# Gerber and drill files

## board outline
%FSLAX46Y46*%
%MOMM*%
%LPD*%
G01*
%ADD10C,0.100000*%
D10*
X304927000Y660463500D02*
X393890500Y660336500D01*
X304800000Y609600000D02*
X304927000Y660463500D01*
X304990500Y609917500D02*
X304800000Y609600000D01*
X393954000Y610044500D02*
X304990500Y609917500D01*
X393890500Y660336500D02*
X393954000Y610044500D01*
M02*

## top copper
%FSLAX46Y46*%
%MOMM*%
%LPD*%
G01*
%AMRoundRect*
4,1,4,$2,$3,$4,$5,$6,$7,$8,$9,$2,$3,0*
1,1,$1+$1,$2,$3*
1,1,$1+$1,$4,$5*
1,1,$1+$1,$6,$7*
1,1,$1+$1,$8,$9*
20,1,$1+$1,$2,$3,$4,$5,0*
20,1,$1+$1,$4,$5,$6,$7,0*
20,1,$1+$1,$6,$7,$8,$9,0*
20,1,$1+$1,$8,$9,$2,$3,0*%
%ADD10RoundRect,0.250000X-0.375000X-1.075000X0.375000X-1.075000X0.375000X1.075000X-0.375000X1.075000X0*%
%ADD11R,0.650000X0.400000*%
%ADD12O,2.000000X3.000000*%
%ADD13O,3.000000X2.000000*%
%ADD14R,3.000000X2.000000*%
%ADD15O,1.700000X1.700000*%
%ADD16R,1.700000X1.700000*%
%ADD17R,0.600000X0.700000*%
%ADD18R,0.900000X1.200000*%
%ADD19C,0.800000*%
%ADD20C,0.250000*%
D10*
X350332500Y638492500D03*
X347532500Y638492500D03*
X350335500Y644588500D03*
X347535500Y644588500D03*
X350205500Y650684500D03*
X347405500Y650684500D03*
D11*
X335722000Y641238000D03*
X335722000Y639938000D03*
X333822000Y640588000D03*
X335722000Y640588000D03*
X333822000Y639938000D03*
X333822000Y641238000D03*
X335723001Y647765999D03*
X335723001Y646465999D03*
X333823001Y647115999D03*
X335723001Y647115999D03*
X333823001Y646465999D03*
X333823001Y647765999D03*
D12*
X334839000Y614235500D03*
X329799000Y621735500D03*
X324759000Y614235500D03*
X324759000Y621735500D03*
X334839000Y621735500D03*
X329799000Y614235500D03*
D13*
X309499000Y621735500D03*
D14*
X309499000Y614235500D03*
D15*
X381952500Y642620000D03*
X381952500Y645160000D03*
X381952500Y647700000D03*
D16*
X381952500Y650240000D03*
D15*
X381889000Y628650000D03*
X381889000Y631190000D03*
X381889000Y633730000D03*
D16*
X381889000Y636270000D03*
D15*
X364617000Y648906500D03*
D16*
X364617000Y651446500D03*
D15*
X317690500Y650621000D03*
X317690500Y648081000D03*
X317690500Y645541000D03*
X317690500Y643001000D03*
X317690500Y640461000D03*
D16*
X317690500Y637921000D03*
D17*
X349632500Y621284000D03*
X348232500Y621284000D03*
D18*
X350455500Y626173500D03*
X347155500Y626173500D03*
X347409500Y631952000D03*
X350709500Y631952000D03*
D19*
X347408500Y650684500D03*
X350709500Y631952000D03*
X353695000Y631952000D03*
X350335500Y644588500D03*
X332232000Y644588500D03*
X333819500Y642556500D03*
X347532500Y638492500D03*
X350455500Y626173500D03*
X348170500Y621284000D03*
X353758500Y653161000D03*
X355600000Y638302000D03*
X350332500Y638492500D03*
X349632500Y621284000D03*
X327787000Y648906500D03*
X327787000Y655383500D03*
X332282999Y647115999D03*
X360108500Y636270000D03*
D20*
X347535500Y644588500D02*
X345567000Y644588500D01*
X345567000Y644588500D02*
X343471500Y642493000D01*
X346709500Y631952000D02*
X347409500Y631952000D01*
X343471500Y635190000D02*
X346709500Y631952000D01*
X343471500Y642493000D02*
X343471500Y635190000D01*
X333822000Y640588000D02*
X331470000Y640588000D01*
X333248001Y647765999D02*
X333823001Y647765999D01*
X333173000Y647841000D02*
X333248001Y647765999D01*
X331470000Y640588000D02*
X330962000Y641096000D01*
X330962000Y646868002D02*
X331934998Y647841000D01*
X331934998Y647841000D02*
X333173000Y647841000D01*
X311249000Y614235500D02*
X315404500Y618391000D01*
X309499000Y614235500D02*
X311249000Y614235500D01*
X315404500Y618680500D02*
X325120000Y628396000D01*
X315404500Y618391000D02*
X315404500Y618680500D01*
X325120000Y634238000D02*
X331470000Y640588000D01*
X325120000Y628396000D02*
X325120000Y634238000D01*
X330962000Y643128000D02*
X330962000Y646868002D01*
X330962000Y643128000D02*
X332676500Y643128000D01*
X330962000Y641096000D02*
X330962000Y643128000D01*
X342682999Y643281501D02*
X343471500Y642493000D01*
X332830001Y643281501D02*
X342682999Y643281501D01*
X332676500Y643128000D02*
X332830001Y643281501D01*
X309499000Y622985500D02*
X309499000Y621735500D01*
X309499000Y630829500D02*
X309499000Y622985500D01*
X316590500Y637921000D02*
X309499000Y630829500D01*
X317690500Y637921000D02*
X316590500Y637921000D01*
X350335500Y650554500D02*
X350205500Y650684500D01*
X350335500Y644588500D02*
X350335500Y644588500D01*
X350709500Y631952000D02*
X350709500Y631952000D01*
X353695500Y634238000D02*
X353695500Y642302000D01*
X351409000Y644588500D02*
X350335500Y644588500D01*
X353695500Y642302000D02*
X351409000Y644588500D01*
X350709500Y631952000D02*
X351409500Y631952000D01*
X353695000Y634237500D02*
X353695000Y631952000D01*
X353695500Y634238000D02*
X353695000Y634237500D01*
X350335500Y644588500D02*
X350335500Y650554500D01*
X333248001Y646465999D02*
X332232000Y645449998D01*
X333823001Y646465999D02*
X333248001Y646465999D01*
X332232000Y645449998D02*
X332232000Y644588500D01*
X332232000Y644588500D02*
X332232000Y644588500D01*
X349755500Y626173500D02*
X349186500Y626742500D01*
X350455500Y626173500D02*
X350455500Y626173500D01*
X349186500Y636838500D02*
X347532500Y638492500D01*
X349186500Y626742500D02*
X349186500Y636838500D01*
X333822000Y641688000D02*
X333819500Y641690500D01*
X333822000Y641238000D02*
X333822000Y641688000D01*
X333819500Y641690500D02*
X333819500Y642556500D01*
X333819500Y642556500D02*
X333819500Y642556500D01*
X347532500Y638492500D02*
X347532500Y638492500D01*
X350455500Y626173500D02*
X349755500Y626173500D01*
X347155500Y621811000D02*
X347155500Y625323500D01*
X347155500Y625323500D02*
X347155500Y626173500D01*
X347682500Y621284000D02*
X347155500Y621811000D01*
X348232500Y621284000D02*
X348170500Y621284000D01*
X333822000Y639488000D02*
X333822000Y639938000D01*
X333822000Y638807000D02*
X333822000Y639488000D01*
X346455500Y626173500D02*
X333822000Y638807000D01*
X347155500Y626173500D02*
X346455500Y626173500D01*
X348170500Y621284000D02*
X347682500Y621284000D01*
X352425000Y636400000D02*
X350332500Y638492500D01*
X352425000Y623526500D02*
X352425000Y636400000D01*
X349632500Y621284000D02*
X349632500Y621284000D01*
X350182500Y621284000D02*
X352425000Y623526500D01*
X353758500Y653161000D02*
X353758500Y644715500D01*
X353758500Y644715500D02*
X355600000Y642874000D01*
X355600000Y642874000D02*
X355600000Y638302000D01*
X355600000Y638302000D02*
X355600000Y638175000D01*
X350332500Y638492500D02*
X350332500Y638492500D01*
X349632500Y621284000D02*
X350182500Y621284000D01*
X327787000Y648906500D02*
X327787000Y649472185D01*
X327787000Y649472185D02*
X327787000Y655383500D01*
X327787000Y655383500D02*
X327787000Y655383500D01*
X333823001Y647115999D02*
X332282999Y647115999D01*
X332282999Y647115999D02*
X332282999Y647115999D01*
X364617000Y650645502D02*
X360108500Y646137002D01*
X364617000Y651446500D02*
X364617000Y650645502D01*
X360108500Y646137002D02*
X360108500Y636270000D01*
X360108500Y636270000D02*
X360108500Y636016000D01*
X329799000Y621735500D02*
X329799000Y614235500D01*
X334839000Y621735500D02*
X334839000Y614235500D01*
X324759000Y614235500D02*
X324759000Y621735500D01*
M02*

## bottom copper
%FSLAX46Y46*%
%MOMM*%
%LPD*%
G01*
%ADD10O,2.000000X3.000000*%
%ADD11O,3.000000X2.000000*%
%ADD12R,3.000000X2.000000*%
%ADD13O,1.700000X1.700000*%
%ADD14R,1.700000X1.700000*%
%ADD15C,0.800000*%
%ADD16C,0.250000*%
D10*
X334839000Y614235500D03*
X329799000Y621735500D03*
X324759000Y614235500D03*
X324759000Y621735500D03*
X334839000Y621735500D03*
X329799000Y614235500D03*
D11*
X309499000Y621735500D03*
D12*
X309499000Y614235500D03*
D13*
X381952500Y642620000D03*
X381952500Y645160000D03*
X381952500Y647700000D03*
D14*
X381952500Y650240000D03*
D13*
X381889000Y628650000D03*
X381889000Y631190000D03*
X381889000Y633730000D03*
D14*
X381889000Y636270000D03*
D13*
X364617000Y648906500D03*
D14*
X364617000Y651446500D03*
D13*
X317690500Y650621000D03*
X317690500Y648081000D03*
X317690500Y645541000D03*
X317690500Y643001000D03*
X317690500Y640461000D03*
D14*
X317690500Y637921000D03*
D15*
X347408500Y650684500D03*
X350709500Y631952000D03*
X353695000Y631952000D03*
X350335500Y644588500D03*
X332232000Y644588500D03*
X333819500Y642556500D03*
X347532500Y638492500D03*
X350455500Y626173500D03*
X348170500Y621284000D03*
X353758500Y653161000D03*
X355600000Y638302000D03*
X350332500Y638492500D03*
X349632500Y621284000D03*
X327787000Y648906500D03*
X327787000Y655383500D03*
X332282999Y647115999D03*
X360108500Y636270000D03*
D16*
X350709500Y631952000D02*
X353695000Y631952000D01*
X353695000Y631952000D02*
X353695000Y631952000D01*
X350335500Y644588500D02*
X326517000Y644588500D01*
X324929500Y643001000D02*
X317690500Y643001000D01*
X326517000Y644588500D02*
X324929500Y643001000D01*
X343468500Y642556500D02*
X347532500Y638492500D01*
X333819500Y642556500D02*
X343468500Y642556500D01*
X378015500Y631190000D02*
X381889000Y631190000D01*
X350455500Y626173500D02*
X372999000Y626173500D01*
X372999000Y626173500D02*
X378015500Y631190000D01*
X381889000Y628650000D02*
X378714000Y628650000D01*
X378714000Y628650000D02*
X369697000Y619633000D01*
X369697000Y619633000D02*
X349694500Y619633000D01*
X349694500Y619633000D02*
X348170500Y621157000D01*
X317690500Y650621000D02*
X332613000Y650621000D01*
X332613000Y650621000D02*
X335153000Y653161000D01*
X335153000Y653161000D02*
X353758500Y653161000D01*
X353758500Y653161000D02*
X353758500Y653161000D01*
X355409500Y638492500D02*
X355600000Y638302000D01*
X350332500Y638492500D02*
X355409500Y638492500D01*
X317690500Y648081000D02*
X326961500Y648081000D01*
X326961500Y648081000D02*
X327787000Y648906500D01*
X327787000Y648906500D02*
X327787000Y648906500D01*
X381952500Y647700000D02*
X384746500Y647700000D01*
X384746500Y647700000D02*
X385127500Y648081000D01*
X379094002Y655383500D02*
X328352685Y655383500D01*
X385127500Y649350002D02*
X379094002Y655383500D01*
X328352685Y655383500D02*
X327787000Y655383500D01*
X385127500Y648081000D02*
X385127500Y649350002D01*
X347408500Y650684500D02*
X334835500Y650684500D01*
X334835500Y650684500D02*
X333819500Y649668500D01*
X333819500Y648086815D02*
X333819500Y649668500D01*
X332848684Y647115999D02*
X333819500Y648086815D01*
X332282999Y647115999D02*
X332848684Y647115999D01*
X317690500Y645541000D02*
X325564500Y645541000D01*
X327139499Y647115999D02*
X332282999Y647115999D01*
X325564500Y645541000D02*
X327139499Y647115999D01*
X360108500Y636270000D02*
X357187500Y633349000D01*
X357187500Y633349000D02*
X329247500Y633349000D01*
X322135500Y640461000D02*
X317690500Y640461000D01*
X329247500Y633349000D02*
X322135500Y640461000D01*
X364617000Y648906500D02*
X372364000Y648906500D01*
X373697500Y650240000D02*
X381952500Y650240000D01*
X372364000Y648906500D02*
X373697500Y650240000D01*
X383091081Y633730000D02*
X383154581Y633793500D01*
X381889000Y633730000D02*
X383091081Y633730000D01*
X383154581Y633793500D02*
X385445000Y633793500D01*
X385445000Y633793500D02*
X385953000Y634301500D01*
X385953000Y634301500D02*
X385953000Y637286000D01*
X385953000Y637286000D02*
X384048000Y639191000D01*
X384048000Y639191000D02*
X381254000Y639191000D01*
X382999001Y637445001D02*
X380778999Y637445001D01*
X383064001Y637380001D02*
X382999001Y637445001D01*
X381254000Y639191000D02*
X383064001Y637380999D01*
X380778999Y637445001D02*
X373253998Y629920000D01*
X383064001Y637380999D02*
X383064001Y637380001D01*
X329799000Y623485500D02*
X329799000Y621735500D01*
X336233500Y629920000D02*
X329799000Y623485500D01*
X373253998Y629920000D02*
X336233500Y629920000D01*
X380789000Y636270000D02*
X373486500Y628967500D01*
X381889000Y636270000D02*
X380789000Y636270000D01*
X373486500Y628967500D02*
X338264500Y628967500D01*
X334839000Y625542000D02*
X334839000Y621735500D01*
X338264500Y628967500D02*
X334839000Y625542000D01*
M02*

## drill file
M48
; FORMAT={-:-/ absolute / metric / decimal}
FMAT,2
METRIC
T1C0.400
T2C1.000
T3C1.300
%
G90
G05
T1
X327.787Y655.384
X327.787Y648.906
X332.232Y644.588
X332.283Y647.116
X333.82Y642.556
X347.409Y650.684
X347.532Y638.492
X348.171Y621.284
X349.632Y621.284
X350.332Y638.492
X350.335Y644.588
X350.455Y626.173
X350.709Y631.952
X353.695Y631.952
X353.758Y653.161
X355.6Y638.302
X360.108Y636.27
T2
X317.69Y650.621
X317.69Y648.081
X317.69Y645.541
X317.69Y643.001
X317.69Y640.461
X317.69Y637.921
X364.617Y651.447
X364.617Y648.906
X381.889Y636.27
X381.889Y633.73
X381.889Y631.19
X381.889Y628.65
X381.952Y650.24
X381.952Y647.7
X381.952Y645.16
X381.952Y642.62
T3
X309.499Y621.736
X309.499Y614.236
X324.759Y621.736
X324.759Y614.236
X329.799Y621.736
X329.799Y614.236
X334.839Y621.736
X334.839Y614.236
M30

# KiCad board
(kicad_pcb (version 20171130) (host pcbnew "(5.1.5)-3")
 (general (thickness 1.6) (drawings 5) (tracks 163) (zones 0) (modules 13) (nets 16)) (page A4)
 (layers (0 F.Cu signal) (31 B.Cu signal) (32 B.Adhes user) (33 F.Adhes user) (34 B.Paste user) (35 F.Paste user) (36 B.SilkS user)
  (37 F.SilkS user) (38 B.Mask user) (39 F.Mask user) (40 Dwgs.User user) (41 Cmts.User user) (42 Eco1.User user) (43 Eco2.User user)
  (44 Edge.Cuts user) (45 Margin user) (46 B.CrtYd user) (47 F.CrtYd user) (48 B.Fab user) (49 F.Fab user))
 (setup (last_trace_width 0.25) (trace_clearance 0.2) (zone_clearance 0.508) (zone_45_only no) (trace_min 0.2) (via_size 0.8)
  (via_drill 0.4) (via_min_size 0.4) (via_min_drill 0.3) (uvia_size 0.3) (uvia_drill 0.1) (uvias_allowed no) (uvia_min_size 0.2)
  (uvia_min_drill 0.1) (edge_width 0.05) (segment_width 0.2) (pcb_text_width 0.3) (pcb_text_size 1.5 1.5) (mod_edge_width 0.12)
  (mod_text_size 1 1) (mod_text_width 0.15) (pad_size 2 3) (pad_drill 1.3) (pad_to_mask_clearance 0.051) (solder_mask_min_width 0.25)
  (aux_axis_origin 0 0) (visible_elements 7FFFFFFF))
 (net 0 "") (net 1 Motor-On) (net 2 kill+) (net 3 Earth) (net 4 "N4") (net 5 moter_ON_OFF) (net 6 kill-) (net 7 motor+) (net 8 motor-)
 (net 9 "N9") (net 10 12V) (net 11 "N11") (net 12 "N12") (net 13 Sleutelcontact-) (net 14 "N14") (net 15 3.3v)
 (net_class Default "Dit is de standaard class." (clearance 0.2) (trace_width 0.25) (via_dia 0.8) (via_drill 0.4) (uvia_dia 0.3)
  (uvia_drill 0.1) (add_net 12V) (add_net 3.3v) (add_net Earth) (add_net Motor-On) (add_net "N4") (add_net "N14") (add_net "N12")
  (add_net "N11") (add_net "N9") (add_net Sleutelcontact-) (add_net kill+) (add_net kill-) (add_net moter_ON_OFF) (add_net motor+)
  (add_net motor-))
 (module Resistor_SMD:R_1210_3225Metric (layer F.Cu) (at 348.9325 -638.4925)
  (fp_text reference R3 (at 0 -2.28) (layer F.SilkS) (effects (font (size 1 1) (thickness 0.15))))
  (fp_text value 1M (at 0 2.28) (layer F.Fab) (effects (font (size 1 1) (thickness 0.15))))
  (pad 2 smd roundrect (at 1.4 0) (size 1.25 2.65) (layers F.Cu F.Paste F.Mask) (roundrect_rratio 0.2) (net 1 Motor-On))
  (pad 1 smd roundrect (at -1.4 0) (size 1.25 2.65) (layers F.Cu F.Paste F.Mask) (roundrect_rratio 0.2) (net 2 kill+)))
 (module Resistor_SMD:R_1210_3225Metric (layer F.Cu) (at 348.9355 -644.5885)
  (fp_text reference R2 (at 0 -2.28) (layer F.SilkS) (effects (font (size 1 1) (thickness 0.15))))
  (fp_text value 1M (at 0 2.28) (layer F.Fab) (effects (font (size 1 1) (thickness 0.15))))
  (pad 2 smd roundrect (at 1.4 0) (size 1.25 2.65) (layers F.Cu F.Paste F.Mask) (roundrect_rratio 0.2) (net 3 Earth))
  (pad 1 smd roundrect (at -1.4 0) (size 1.25 2.65) (layers F.Cu F.Paste F.Mask) (roundrect_rratio 0.2) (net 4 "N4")))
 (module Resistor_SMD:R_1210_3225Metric (layer F.Cu) (at 348.8055 -650.6845)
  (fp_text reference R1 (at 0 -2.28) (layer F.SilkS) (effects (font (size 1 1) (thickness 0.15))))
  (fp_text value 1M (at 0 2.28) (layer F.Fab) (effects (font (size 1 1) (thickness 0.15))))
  (pad 2 smd roundrect (at 1.4 0) (size 1.25 2.65) (layers F.Cu F.Paste F.Mask) (roundrect_rratio 0.2) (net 3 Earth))
  (pad 1 smd roundrect (at -1.4 0) (size 1.25 2.65) (layers F.Cu F.Paste F.Mask) (roundrect_rratio 0.2) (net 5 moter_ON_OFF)))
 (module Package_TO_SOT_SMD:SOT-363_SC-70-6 (layer F.Cu) (at 334.772 -640.588)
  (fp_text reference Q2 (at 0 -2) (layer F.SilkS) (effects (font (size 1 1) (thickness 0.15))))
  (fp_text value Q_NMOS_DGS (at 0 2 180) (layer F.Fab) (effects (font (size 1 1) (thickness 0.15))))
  (pad 6 smd rect (at 0.95 -0.65) (size 0.65 0.4) (layers F.Cu F.Paste F.Mask))
  (pad 4 smd rect (at 0.95 0.65) (size 0.65 0.4) (layers F.Cu F.Paste F.Mask))
  (pad 2 smd rect (at -0.95 0) (size 0.65 0.4) (layers F.Cu F.Paste F.Mask) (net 4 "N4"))
  (pad 5 smd rect (at 0.95 0) (size 0.65 0.4) (layers F.Cu F.Paste F.Mask))
  (pad 3 smd rect (at -0.95 0.65) (size 0.65 0.4) (layers F.Cu F.Paste F.Mask) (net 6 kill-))
  (pad 1 smd rect (at -0.95 -0.65) (size 0.65 0.4) (layers F.Cu F.Paste F.Mask) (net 2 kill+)))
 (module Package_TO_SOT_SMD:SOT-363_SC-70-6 (layer F.Cu) (at 334.773001 -647.115999)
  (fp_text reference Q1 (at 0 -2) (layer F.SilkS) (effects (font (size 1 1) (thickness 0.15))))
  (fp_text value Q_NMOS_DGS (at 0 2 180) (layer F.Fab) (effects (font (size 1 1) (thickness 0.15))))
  (pad 6 smd rect (at 0.95 -0.65) (size 0.65 0.4) (layers F.Cu F.Paste F.Mask))
  (pad 4 smd rect (at 0.95 0.65) (size 0.65 0.4) (layers F.Cu F.Paste F.Mask))
  (pad 2 smd rect (at -0.95 0) (size 0.65 0.4) (layers F.Cu F.Paste F.Mask) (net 5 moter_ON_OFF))
  (pad 5 smd rect (at 0.95 0) (size 0.65 0.4) (layers F.Cu F.Paste F.Mask))
  (pad 3 smd rect (at -0.95 0.65) (size 0.65 0.4) (layers F.Cu F.Paste F.Mask) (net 3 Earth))
  (pad 1 smd rect (at -0.95 -0.65) (size 0.65 0.4) (layers F.Cu F.Paste F.Mask) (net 4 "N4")))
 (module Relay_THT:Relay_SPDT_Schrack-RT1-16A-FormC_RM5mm (layer F.Cu) (at 309.499 -614.2355)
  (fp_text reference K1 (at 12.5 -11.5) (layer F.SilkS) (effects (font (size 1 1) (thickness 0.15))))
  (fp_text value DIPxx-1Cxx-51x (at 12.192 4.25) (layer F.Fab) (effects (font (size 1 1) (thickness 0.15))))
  (pad 14 thru_hole oval (at 25.34 0 180) (size 2 3) (drill 1.3) (layers *.Cu *.Mask) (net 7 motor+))
  (pad 7 thru_hole oval (at 20.3 -7.5 180) (size 2 3) (drill 1.3) (layers *.Cu *.Mask) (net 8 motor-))
  (pad 1 thru_hole oval (at 15.26 0 180) (size 2 3) (drill 1.3) (layers *.Cu *.Mask Eco1.User) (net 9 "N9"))
  (pad 1 thru_hole oval (at 15.26 -7.5 180) (size 2 3) (drill 1.3) (layers *.Cu *.Mask) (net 9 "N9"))
  (pad 14 thru_hole oval (at 25.34 -7.5 180) (size 2 3) (drill 1.3) (layers *.Cu *.Mask) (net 7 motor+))
  (pad 7 thru_hole oval (at 20.3 0 180) (size 2 3) (drill 1.3) (layers *.Cu *.Mask) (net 8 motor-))
  (pad 6 thru_hole oval (at 0 -7.5 180) (size 3 2) (drill 1.3) (layers *.Cu *.Mask) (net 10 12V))
  (pad 2 thru_hole rect (at 0 0 180) (size 3 2) (drill 1.3) (layers *.Cu *.Mask Eco2.User) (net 4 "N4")))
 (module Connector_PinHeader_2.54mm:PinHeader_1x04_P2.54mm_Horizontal (layer F.Cu) (at 381.9525 -650.24)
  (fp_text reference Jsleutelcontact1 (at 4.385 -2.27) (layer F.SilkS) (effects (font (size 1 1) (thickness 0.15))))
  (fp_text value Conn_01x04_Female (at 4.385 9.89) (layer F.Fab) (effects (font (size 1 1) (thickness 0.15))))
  (pad 4 thru_hole oval (at 0 7.62) (size 1.7 1.7) (drill 1) (layers *.Cu *.Mask) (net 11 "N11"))
  (pad 3 thru_hole oval (at 0 5.08) (size 1.7 1.7) (drill 1) (layers *.Cu *.Mask) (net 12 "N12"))
  (pad 2 thru_hole oval (at 0 2.54) (size 1.7 1.7) (drill 1) (layers *.Cu *.Mask) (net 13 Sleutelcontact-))
  (pad 1 thru_hole rect (at 0 0) (size 1.7 1.7) (drill 1) (layers *.Cu *.Mask) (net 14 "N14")))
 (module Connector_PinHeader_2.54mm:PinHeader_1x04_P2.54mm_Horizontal (layer F.Cu) (at 381.889 -636.27)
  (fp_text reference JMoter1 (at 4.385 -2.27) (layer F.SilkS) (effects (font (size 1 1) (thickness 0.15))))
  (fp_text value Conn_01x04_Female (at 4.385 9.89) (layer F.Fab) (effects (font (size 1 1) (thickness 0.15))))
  (pad 4 thru_hole oval (at 0 7.62) (size 1.7 1.7) (drill 1) (layers *.Cu *.Mask) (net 6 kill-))
  (pad 3 thru_hole oval (at 0 5.08) (size 1.7 1.7) (drill 1) (layers *.Cu *.Mask) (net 2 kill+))
  (pad 2 thru_hole oval (at 0 2.54) (size 1.7 1.7) (drill 1) (layers *.Cu *.Mask) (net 8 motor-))
  (pad 1 thru_hole rect (at 0 0) (size 1.7 1.7) (drill 1) (layers *.Cu *.Mask) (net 7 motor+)))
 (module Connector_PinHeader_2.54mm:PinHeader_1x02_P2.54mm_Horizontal (layer F.Cu) (at 364.617 -651.4465)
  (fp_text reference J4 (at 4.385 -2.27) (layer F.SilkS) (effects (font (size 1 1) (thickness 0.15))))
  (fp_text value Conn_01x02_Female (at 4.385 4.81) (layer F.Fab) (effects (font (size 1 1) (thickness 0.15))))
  (pad 2 thru_hole oval (at 0 2.54) (size 1.7 1.7) (drill 1) (layers *.Cu *.Mask) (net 14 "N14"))
  (pad 1 thru_hole rect (at 0 0) (size 1.7 1.7) (drill 1) (layers *.Cu *.Mask) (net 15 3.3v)))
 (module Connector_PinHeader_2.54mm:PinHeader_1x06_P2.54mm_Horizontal (layer F.Cu) (at 317.6905 -637.921 180)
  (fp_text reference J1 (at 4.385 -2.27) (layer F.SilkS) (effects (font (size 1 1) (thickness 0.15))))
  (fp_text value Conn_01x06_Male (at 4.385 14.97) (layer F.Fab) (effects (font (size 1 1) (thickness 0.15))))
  (pad 6 thru_hole oval (at 0 12.7 180) (size 1.7 1.7) (drill 1) (layers *.Cu *.Mask) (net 1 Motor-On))
  (pad 5 thru_hole oval (at 0 10.16 180) (size 1.7 1.7) (drill 1) (layers *.Cu *.Mask) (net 13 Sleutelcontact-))
  (pad 4 thru_hole oval (at 0 7.62 180) (size 1.7 1.7) (drill 1) (layers *.Cu *.Mask) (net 5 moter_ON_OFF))
  (pad 3 thru_hole oval (at 0 5.08 180) (size 1.7 1.7) (drill 1) (layers *.Cu *.Mask) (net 3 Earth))
  (pad 2 thru_hole oval (at 0 2.54 180) (size 1.7 1.7) (drill 1) (layers *.Cu *.Mask) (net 15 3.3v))
  (pad 1 thru_hole rect (at 0 0 180) (size 1.7 1.7) (drill 1) (layers *.Cu *.Mask) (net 10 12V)))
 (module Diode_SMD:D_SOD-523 (layer F.Cu) (at 348.9325 -621.284 180)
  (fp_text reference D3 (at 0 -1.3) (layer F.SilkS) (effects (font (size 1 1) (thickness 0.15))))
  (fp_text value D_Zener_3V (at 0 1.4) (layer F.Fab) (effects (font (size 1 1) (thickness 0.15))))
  (pad 1 smd rect (at -0.7 0) (size 0.6 0.7) (layers F.Cu F.Paste F.Mask) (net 1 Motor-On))
  (pad 2 smd rect (at 0.7 0) (size 0.6 0.7) (layers F.Cu F.Paste F.Mask) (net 6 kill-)))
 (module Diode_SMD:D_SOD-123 (layer F.Cu) (at 348.8055 -626.1735)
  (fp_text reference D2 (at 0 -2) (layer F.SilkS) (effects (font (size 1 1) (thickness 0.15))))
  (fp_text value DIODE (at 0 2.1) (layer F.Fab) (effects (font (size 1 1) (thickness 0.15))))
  (pad 2 smd rect (at 1.65 0) (size 0.9 1.2) (layers F.Cu F.Paste F.Mask) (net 2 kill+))
  (pad 1 smd rect (at -1.65 0) (size 0.9 1.2) (layers F.Cu F.Paste F.Mask) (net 6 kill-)))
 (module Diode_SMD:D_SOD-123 (layer F.Cu) (at 349.0595 -631.952 180)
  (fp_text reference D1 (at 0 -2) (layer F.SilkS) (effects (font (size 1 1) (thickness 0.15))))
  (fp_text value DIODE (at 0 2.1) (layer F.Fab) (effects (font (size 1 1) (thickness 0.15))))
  (pad 2 smd rect (at 1.65 0 180) (size 0.9 1.2) (layers F.Cu F.Paste F.Mask) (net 4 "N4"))
  (pad 1 smd rect (at -1.65 0 180) (size 0.9 1.2) (layers F.Cu F.Paste F.Mask) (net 3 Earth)))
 (gr_line (start 304.927 -660.4635) (end 393.8905 -660.3365) (layer Edge.Cuts) (width 0.1))
 (gr_line (start 304.8 -609.6) (end 304.927 -660.4635) (layer Edge.Cuts) (width 0.1))
 (gr_line (start 304.9905 -609.9175) (end 304.8 -609.6) (layer Edge.Cuts) (width 0.1))
 (gr_line (start 393.954 -610.0445) (end 304.9905 -609.9175) (layer Edge.Cuts) (width 0.1))
 (gr_line (start 393.8905 -660.3365) (end 393.954 -610.0445) (layer Edge.Cuts) (width 0.1))
 (via (at 347.4085 -650.6845) (size 0.8) (drill 0.4) (layers F.Cu B.Cu) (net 5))
 (segment (start 347.5355 -644.5885) (end 345.567 -644.5885) (width 0.25) (layer F.Cu) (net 4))
 (segment (start 345.567 -644.5885) (end 343.4715 -642.493) (width 0.25) (layer F.Cu) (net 4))
 (segment (start 346.7095 -631.952) (end 347.4095 -631.952) (width 0.25) (layer F.Cu) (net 4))
 (segment (start 343.4715 -635.19) (end 346.7095 -631.952) (width 0.25) (layer F.Cu) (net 4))
 (segment (start 343.4715 -642.493) (end 343.4715 -635.19) (width 0.25) (layer F.Cu) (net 4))
 (segment (start 333.822 -640.588) (end 331.47 -640.588) (width 0.25) (layer F.Cu) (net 4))
 (segment (start 333.248001 -647.765999) (end 333.823001 -647.765999) (width 0.25) (layer F.Cu) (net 4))
 (segment (start 333.173 -647.841) (end 333.248001 -647.765999) (width 0.25) (layer F.Cu) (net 4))
 (segment (start 331.47 -640.588) (end 330.962 -641.096) (width 0.25) (layer F.Cu) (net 4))
 (segment (start 330.962 -646.868002) (end 331.934998 -647.841) (width 0.25) (layer F.Cu) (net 4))
 (segment (start 331.934998 -647.841) (end 333.173 -647.841) (width 0.25) (layer F.Cu) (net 4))
 (segment (start 311.249 -614.2355) (end 315.4045 -618.391) (width 0.25) (layer F.Cu) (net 4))
 (segment (start 309.499 -614.2355) (end 311.249 -614.2355) (width 0.25) (layer F.Cu) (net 4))
 (segment (start 315.4045 -618.6805) (end 325.12 -628.396) (width 0.25) (layer F.Cu) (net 4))
 (segment (start 315.4045 -618.391) (end 315.4045 -618.6805) (width 0.25) (layer F.Cu) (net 4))
 (segment (start 325.12 -634.238) (end 331.47 -640.588) (width 0.25) (layer F.Cu) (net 4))
 (segment (start 325.12 -628.396) (end 325.12 -634.238) (width 0.25) (layer F.Cu) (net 4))
 (segment (start 330.962 -643.128) (end 330.962 -646.868002) (width 0.25) (layer F.Cu) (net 4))
 (segment (start 330.962 -643.128) (end 332.6765 -643.128) (width 0.25) (layer F.Cu) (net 4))
 (segment (start 330.962 -641.096) (end 330.962 -643.128) (width 0.25) (layer F.Cu) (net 4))
 (segment (start 342.682999 -643.281501) (end 343.4715 -642.493) (width 0.25) (layer F.Cu) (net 4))
 (segment (start 332.830001 -643.281501) (end 342.682999 -643.281501) (width 0.25) (layer F.Cu) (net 4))
 (segment (start 332.6765 -643.128) (end 332.830001 -643.281501) (width 0.25) (layer F.Cu) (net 4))
 (segment (start 309.499 -622.9855) (end 309.499 -621.7355) (width 0.25) (layer F.Cu) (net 10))
 (segment (start 309.499 -630.8295) (end 309.499 -622.9855) (width 0.25) (layer F.Cu) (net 10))
 (segment (start 316.5905 -637.921) (end 309.499 -630.8295) (width 0.25) (layer F.Cu) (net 10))
 (segment (start 317.6905 -637.921) (end 316.5905 -637.921) (width 0.25) (layer F.Cu) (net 10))
 (segment (start 350.3355 -650.5545) (end 350.2055 -650.6845) (width 0.25) (layer F.Cu) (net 3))
 (segment (start 350.3355 -644.5885) (end 350.3355 -644.5885) (width 0.25) (layer F.Cu) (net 3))
 (segment (start 350.7095 -631.952) (end 350.7095 -631.952) (width 0.25) (layer F.Cu) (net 3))
 (segment (start 353.6955 -634.238) (end 353.6955 -642.302) (width 0.25) (layer F.Cu) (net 3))
 (segment (start 351.409 -644.5885) (end 350.3355 -644.5885) (width 0.25) (layer F.Cu) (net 3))
 (segment (start 353.6955 -642.302) (end 351.409 -644.5885) (width 0.25) (layer F.Cu) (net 3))
 (segment (start 350.7095 -631.952) (end 351.4095 -631.952) (width 0.25) (layer F.Cu) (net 3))
 (via (at 350.7095 -631.952) (size 0.8) (drill 0.4) (layers F.Cu B.Cu) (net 3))
 (segment (start 350.7095 -631.952) (end 353.695 -631.952) (width 0.25) (layer B.Cu) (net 3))
 (segment (start 353.695 -631.952) (end 353.695 -631.952) (width 0.25) (layer B.Cu) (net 3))
 (via (at 353.695 -631.952) (size 0.8) (drill 0.4) (layers F.Cu B.Cu) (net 3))
 (segment (start 353.695 -634.2375) (end 353.695 -631.952) (width 0.25) (layer F.Cu) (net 3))
 (segment (start 353.6955 -634.238) (end 353.695 -634.2375) (width 0.25) (layer F.Cu) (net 3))
 (segment (start 350.3355 -644.5885) (end 350.3355 -650.5545) (width 0.25) (layer F.Cu) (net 3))
 (via (at 350.3355 -644.5885) (size 0.8) (drill 0.4) (layers F.Cu B.Cu) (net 3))
 (segment (start 350.3355 -644.5885) (end 326.517 -644.5885) (width 0.25) (layer B.Cu) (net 3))
 (segment (start 324.9295 -643.001) (end 317.6905 -643.001) (width 0.25) (layer B.Cu) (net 3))
 (segment (start 326.517 -644.5885) (end 324.9295 -643.001) (width 0.25) (layer B.Cu) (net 3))
 (segment (start 333.248001 -646.465999) (end 332.232 -645.449998) (width 0.25) (layer F.Cu) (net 3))
 (segment (start 333.823001 -646.465999) (end 333.248001 -646.465999) (width 0.25) (layer F.Cu) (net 3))
 (segment (start 332.232 -645.449998) (end 332.232 -644.5885) (width 0.25) (layer F.Cu) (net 3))
 (segment (start 332.232 -644.5885) (end 332.232 -644.5885) (width 0.25) (layer F.Cu) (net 3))
 (via (at 332.232 -644.5885) (size 0.8) (drill 0.4) (layers F.Cu B.Cu) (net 3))
 (segment (start 349.7555 -626.1735) (end 349.1865 -626.7425) (width 0.25) (layer F.Cu) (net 2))
 (segment (start 350.4555 -626.1735) (end 350.4555 -626.1735) (width 0.25) (layer F.Cu) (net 2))
 (segment (start 349.1865 -636.8385) (end 347.5325 -638.4925) (width 0.25) (layer F.Cu) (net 2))
 (segment (start 349.1865 -626.7425) (end 349.1865 -636.8385) (width 0.25) (layer F.Cu) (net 2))
 (segment (start 333.822 -641.688) (end 333.8195 -641.6905) (width 0.25) (layer F.Cu) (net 2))
 (segment (start 333.822 -641.238) (end 333.822 -641.688) (width 0.25) (layer F.Cu) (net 2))
 (segment (start 333.8195 -641.6905) (end 333.8195 -642.5565) (width 0.25) (layer F.Cu) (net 2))
 (segment (start 333.8195 -642.5565) (end 333.8195 -642.5565) (width 0.25) (layer F.Cu) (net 2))
 (via (at 333.8195 -642.5565) (size 0.8) (drill 0.4) (layers F.Cu B.Cu) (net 2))
 (segment (start 347.5325 -638.4925) (end 347.5325 -638.4925) (width 0.25) (layer F.Cu) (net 2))
 (via (at 347.5325 -638.4925) (size 0.8) (drill 0.4) (layers F.Cu B.Cu) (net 2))
 (segment (start 343.4685 -642.5565) (end 347.5325 -638.4925) (width 0.25) (layer B.Cu) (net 2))
 (segment (start 333.8195 -642.5565) (end 343.4685 -642.5565) (width 0.25) (layer B.Cu) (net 2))
 (segment (start 350.4555 -626.1735) (end 349.7555 -626.1735) (width 0.25) (layer F.Cu) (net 2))
 (via (at 350.4555 -626.1735) (size 0.8) (drill 0.4) (layers F.Cu B.Cu) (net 2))
 (segment (start 378.0155 -631.19) (end 381.889 -631.19) (width 0.25) (layer B.Cu) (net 2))
 (segment (start 350.4555 -626.1735) (end 372.999 -626.1735) (width 0.25) (layer B.Cu) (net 2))
 (segment (start 372.999 -626.1735) (end 378.0155 -631.19) (width 0.25) (layer B.Cu) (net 2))
 (segment (start 347.1555 -621.811) (end 347.1555 -625.3235) (width 0.25) (layer F.Cu) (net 6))
 (segment (start 347.1555 -625.3235) (end 347.1555 -626.1735) (width 0.25) (layer F.Cu) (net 6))
 (segment (start 347.6825 -621.284) (end 347.1555 -621.811) (width 0.25) (layer F.Cu) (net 6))
 (segment (start 348.2325 -621.284) (end 348.1705 -621.284) (width 0.25) (layer F.Cu) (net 6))
 (segment (start 333.822 -639.488) (end 333.822 -639.938) (width 0.25) (layer F.Cu) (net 6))
 (segment (start 333.822 -638.807) (end 333.822 -639.488) (width 0.25) (layer F.Cu) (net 6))
 (segment (start 346.4555 -626.1735) (end 333.822 -638.807) (width 0.25) (layer F.Cu) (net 6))
 (segment (start 347.1555 -626.1735) (end 346.4555 -626.1735) (width 0.25) (layer F.Cu) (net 6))
 (segment (start 381.889 -628.65) (end 378.714 -628.65) (width 0.25) (layer B.Cu) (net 6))
 (segment (start 378.714 -628.65) (end 369.697 -619.633) (width 0.25) (layer B.Cu) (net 6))
 (segment (start 369.697 -619.633) (end 349.6945 -619.633) (width 0.25) (layer B.Cu) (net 6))
 (segment (start 349.6945 -619.633) (end 348.1705 -621.157) (width 0.25) (layer B.Cu) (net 6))
 (segment (start 348.1705 -621.284) (end 347.6825 -621.284) (width 0.25) (layer F.Cu) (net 6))
 (via (at 348.1705 -621.284) (size 0.8) (drill 0.4) (layers F.Cu B.Cu) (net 6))
 (segment (start 352.425 -636.4) (end 350.3325 -638.4925) (width 0.25) (layer F.Cu) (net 1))
 (segment (start 352.425 -623.5265) (end 352.425 -636.4) (width 0.25) (layer F.Cu) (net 1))
 (segment (start 349.6325 -621.284) (end 349.6325 -621.284) (width 0.25) (layer F.Cu) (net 1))
 (segment (start 350.1825 -621.284) (end 352.425 -623.5265) (width 0.25) (layer F.Cu) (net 1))
 (segment (start 317.6905 -650.621) (end 332.613 -650.621) (width 0.25) (layer B.Cu) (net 1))
 (segment (start 332.613 -650.621) (end 335.153 -653.161) (width 0.25) (layer B.Cu) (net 1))
 (segment (start 335.153 -653.161) (end 353.7585 -653.161) (width 0.25) (layer B.Cu) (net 1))
 (segment (start 353.7585 -653.161) (end 353.7585 -653.161) (width 0.25) (layer B.Cu) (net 1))
 (via (at 353.7585 -653.161) (size 0.8) (drill 0.4) (layers F.Cu B.Cu) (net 1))
 (segment (start 353.7585 -653.161) (end 353.7585 -644.7155) (width 0.25) (layer F.Cu) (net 1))
 (segment (start 353.7585 -644.7155) (end 355.6 -642.874) (width 0.25) (layer F.Cu) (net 1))
 (segment (start 355.6 -642.874) (end 355.6 -638.302) (width 0.25) (layer F.Cu) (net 1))
 (segment (start 355.6 -638.302) (end 355.6 -638.175) (width 0.25) (layer F.Cu) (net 1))
 (via (at 355.6 -638.302) (size 0.8) (drill 0.4) (layers F.Cu B.Cu) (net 1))
 (segment (start 350.3325 -638.4925) (end 350.3325 -638.4925) (width 0.25) (layer F.Cu) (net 1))
 (via (at 350.3325 -638.4925) (size 0.8) (drill 0.4) (layers F.Cu B.Cu) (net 1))
 (segment (start 355.4095 -638.4925) (end 355.6 -638.302) (width 0.25) (layer B.Cu) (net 1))
 (segment (start 350.3325 -638.4925) (end 355.4095 -638.4925) (width 0.25) (layer B.Cu) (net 1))
 (segment (start 349.6325 -621.284) (end 350.1825 -621.284) (width 0.25) (layer F.Cu) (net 1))
 (via (at 349.6325 -621.284) (size 0.8) (drill 0.4) (layers F.Cu B.Cu) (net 1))
 (segment (start 317.6905 -648.081) (end 326.9615 -648.081) (width 0.25) (layer B.Cu) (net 13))
 (segment (start 326.9615 -648.081) (end 327.787 -648.9065) (width 0.25) (layer B.Cu) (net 13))
 (segment (start 327.787 -648.9065) (end 327.787 -648.9065) (width 0.25) (layer B.Cu) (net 13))
 (via (at 327.787 -648.9065) (size 0.8) (drill 0.4) (layers F.Cu B.Cu) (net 13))
 (segment (start 327.787 -648.9065) (end 327.787 -649.472185) (width 0.25) (layer F.Cu) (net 13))
 (segment (start 327.787 -649.472185) (end 327.787 -655.3835) (width 0.25) (layer F.Cu) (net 13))
 (segment (start 327.787 -655.3835) (end 327.787 -655.3835) (width 0.25) (layer F.Cu) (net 13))
 (via (at 327.787 -655.3835) (size 0.8) (drill 0.4) (layers F.Cu B.Cu) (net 13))
 (segment (start 381.9525 -647.7) (end 384.7465 -647.7) (width 0.25) (layer B.Cu) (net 13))
 (segment (start 384.7465 -647.7) (end 385.1275 -648.081) (width 0.25) (layer B.Cu) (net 13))
 (segment (start 379.094002 -655.3835) (end 328.352685 -655.3835) (width 0.25) (layer B.Cu) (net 13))
 (segment (start 385.1275 -649.350002) (end 379.094002 -655.3835) (width 0.25) (layer B.Cu) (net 13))
 (segment (start 328.352685 -655.3835) (end 327.787 -655.3835) (width 0.25) (layer B.Cu) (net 13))
 (segment (start 385.1275 -648.081) (end 385.1275 -649.350002) (width 0.25) (layer B.Cu) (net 13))
 (segment (start 347.4085 -650.6845) (end 334.8355 -650.6845) (width 0.25) (layer B.Cu) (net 5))
 (segment (start 334.8355 -650.6845) (end 333.8195 -649.6685) (width 0.25) (layer B.Cu) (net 5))
 (segment (start 333.823001 -647.115999) (end 332.282999 -647.115999) (width 0.25) (layer F.Cu) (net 5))
 (segment (start 332.282999 -647.115999) (end 332.282999 -647.115999) (width 0.25) (layer F.Cu) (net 5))
 (via (at 332.282999 -647.115999) (size 0.8) (drill 0.4) (layers F.Cu B.Cu) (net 5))
 (segment (start 333.8195 -648.086815) (end 333.8195 -649.6685) (width 0.25) (layer B.Cu) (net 5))
 (segment (start 332.848684 -647.115999) (end 333.8195 -648.086815) (width 0.25) (layer B.Cu) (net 5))
 (segment (start 332.282999 -647.115999) (end 332.848684 -647.115999) (width 0.25) (layer B.Cu) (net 5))
 (segment (start 317.6905 -645.541) (end 325.5645 -645.541) (width 0.25) (layer B.Cu) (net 5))
 (segment (start 327.139499 -647.115999) (end 332.282999 -647.115999) (width 0.25) (layer B.Cu) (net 5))
 (segment (start 325.5645 -645.541) (end 327.139499 -647.115999) (width 0.25) (layer B.Cu) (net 5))
 (segment (start 364.617 -650.645502) (end 360.1085 -646.137002) (width 0.25) (layer F.Cu) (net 15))
 (segment (start 364.617 -651.4465) (end 364.617 -650.645502) (width 0.25) (layer F.Cu) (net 15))
 (segment (start 360.1085 -646.137002) (end 360.1085 -636.27) (width 0.25) (layer F.Cu) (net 15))
 (segment (start 360.1085 -636.27) (end 360.1085 -636.016) (width 0.25) (layer F.Cu) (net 15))
 (via (at 360.1085 -636.27) (size 0.8) (drill 0.4) (layers F.Cu B.Cu) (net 15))
 (segment (start 360.1085 -636.27) (end 357.1875 -633.349) (width 0.25) (layer B.Cu) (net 15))
 (segment (start 357.1875 -633.349) (end 329.2475 -633.349) (width 0.25) (layer B.Cu) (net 15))
 (segment (start 322.1355 -640.461) (end 317.6905 -640.461) (width 0.25) (layer B.Cu) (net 15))
 (segment (start 329.2475 -633.349) (end 322.1355 -640.461) (width 0.25) (layer B.Cu) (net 15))
 (segment (start 364.617 -648.9065) (end 372.364 -648.9065) (width 0.25) (layer B.Cu) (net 14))
 (segment (start 373.6975 -650.24) (end 381.9525 -650.24) (width 0.25) (layer B.Cu) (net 14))
 (segment (start 372.364 -648.9065) (end 373.6975 -650.24) (width 0.25) (layer B.Cu) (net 14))
 (segment (start 329.799 -621.7355) (end 329.799 -614.2355) (width 0.25) (layer F.Cu) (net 8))
 (segment (start 383.091081 -633.73) (end 383.154581 -633.7935) (width 0.25) (layer B.Cu) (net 8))
 (segment (start 381.889 -633.73) (end 383.091081 -633.73) (width 0.25) (layer B.Cu) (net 8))
 (segment (start 383.154581 -633.7935) (end 385.445 -633.7935) (width 0.25) (layer B.Cu) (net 8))
 (segment (start 385.445 -633.7935) (end 385.953 -634.3015) (width 0.25) (layer B.Cu) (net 8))
 (segment (start 385.953 -634.3015) (end 385.953 -637.286) (width 0.25) (layer B.Cu) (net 8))
 (segment (start 385.953 -637.286) (end 384.048 -639.191) (width 0.25) (layer B.Cu) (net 8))
 (segment (start 384.048 -639.191) (end 381.254 -639.191) (width 0.25) (layer B.Cu) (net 8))
 (segment (start 382.999001 -637.445001) (end 380.778999 -637.445001) (width 0.25) (layer B.Cu) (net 8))
 (segment (start 383.064001 -637.380001) (end 382.999001 -637.445001) (width 0.25) (layer B.Cu) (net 8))
 (segment (start 381.254 -639.191) (end 383.064001 -637.380999) (width 0.25) (layer B.Cu) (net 8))
 (segment (start 380.778999 -637.445001) (end 373.253998 -629.92) (width 0.25) (layer B.Cu) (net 8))
 (segment (start 383.064001 -637.380999) (end 383.064001 -637.380001) (width 0.25) (layer B.Cu) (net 8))
 (segment (start 329.799 -623.4855) (end 329.799 -621.7355) (width 0.25) (layer B.Cu) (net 8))
 (segment (start 336.2335 -629.92) (end 329.799 -623.4855) (width 0.25) (layer B.Cu) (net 8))
 (segment (start 373.253998 -629.92) (end 336.2335 -629.92) (width 0.25) (layer B.Cu) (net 8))
 (segment (start 334.839 -621.7355) (end 334.839 -614.2355) (width 0.25) (layer F.Cu) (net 7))
 (segment (start 380.789 -636.27) (end 373.4865 -628.9675) (width 0.25) (layer B.Cu) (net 7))
 (segment (start 381.889 -636.27) (end 380.789 -636.27) (width 0.25) (layer B.Cu) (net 7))
 (segment (start 373.4865 -628.9675) (end 338.2645 -628.9675) (width 0.25) (layer B.Cu) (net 7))
 (segment (start 334.839 -625.542) (end 334.839 -621.7355) (width 0.25) (layer B.Cu) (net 7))
 (segment (start 338.2645 -628.9675) (end 334.839 -625.542) (width 0.25) (layer B.Cu) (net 7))
 (segment (start 324.759 -614.2355) (end 324.759 -621.7355) (width 0.25) (layer F.Cu) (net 9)))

